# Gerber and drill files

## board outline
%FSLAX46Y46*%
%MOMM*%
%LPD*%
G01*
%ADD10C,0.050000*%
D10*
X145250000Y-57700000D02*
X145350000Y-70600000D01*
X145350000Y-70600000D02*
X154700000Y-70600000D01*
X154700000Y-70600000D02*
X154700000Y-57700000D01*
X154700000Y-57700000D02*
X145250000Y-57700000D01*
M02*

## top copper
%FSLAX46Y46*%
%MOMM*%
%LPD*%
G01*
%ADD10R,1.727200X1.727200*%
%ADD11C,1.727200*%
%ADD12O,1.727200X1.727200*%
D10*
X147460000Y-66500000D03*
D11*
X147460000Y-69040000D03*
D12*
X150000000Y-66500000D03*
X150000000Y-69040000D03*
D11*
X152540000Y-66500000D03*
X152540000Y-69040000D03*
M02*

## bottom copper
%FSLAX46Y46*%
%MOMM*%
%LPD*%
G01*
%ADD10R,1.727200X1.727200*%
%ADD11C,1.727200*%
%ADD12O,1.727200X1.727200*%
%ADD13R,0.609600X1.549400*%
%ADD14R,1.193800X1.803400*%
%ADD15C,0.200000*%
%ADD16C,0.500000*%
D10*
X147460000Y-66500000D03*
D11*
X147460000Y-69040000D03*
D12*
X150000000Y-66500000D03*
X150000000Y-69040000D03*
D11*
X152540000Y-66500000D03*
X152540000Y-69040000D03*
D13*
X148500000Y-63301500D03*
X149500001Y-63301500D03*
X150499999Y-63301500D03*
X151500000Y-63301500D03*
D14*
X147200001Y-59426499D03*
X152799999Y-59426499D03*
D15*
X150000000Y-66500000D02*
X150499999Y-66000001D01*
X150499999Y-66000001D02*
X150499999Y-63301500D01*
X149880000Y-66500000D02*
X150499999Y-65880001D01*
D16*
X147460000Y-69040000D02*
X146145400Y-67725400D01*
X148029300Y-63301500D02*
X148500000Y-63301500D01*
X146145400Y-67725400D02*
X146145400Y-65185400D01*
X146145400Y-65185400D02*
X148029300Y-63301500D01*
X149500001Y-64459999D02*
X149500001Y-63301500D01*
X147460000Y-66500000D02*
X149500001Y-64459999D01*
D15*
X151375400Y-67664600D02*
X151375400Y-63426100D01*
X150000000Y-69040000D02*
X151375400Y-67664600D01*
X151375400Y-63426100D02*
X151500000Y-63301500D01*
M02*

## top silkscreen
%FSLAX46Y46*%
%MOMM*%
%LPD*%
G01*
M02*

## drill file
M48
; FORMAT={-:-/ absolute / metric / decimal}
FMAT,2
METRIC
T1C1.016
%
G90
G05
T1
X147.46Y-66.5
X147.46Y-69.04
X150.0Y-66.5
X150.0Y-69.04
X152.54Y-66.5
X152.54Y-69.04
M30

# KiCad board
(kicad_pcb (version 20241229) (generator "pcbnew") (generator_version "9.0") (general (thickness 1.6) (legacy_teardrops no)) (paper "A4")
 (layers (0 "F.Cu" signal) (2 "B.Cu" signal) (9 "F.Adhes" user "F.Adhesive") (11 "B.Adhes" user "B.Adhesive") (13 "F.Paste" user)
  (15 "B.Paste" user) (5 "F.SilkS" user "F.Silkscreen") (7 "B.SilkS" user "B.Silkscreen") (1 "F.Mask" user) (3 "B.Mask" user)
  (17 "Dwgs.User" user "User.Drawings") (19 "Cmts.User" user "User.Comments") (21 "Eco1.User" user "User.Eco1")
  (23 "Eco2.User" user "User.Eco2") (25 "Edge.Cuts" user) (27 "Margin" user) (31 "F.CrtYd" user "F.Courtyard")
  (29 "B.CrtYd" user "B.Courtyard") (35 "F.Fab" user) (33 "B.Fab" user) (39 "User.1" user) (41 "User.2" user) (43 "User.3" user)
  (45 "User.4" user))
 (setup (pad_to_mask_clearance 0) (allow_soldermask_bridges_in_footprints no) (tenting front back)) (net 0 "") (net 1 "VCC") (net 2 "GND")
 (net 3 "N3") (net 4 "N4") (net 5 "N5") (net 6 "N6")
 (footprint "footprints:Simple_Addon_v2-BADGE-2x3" (layer "F.Cu") (at 149.94 67.75)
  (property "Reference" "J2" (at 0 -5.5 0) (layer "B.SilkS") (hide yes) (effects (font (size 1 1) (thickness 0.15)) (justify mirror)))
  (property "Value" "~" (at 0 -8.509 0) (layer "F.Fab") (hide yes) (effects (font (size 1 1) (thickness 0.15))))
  (pad "1" thru_hole rect (at -2.48 -1.25 270) (size 1.7272 1.7272) (drill 1.016) (layers "*.Cu" "*.Mask") (remove_unused_layers no)
   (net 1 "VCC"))
  (pad "2" thru_hole circle (at -2.48 1.29 270) (size 1.7272 1.7272) (drill 1.016) (layers "*.Cu" "*.Mask") (remove_unused_layers no)
   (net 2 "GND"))
  (pad "3" thru_hole oval (at 0.06 -1.25 270) (size 1.7272 1.7272) (drill 1.016) (layers "*.Cu" "*.Mask") (remove_unused_layers no)
   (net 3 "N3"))
  (pad "4" thru_hole oval (at 0.06 1.29 270) (size 1.7272 1.7272) (drill 1.016) (layers "*.Cu" "*.Mask") (remove_unused_layers no)
   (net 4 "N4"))
  (pad "5" thru_hole circle (at 2.6 -1.25 270) (size 1.7272 1.7272) (drill 1.016) (layers "*.Cu" "*.Mask") (remove_unused_layers no)
   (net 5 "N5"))
  (pad "6" thru_hole circle (at 2.6 1.29 270) (size 1.7272 1.7272) (drill 1.016) (layers "*.Cu" "*.Mask") (remove_unused_layers no)
   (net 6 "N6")))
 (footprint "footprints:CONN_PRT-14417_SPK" (layer "B.Cu") (at 150 61.2)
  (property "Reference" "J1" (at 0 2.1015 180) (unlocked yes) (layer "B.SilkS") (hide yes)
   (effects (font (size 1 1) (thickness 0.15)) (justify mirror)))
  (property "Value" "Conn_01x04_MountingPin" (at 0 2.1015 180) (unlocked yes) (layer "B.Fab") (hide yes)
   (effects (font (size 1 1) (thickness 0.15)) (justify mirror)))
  (pad "1" smd rect (at -1.5 2.1015) (size 0.6096 1.5494) (layers "B.Cu" "B.Mask" "B.Paste") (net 2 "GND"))
  (pad "2" smd rect (at -0.499999 2.1015) (size 0.6096 1.5494) (layers "B.Cu" "B.Mask" "B.Paste") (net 1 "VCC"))
  (pad "3" smd rect (at 0.499999 2.1015) (size 0.6096 1.5494) (layers "B.Cu" "B.Mask" "B.Paste") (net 3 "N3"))
  (pad "4" smd rect (at 1.5 2.1015) (size 0.6096 1.5494) (layers "B.Cu" "B.Mask" "B.Paste") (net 4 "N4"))
  (pad "5" smd rect (at -2.799999 -1.773501) (size 1.1938 1.8034) (layers "B.Cu" "B.Mask" "B.Paste"))
  (pad "6" smd rect (at 2.799999 -1.773501) (size 1.1938 1.8034) (layers "B.Cu" "B.Mask" "B.Paste")))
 (gr_line (start 145.25 57.7) (end 145.35 70.6) (stroke (width 0.05) (type default)) (layer "Edge.Cuts"))
 (gr_line (start 145.35 70.6) (end 154.7 70.6) (stroke (width 0.05) (type default)) (layer "Edge.Cuts"))
 (gr_line (start 154.7 70.6) (end 154.7 57.7) (stroke (width 0.05) (type default)) (layer "Edge.Cuts"))
 (gr_line (start 154.7 57.7) (end 145.25 57.7) (stroke (width 0.05) (type default)) (layer "Edge.Cuts"))
 (segment (start 150 66.5) (end 150.499999 66.000001) (width 0.2) (layer "B.Cu") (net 3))
 (segment (start 150.499999 66.000001) (end 150.499999 63.3015) (width 0.2) (layer "B.Cu") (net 3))
 (segment (start 149.88 66.5) (end 150.499999 65.880001) (width 0.2) (layer "B.Cu") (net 3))
 (segment (start 147.46 69.04) (end 146.1454 67.7254) (width 0.5) (layer "B.Cu") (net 2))
 (segment (start 148.0293 63.3015) (end 148.5 63.3015) (width 0.5) (layer "B.Cu") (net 2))
 (segment (start 146.1454 67.7254) (end 146.1454 65.1854) (width 0.5) (layer "B.Cu") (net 2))
 (segment (start 146.1454 65.1854) (end 148.0293 63.3015) (width 0.5) (layer "B.Cu") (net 2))
 (segment (start 149.500001 64.459999) (end 149.500001 63.3015) (width 0.5) (layer "B.Cu") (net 1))
 (segment (start 147.46 66.5) (end 149.500001 64.459999) (width 0.5) (layer "B.Cu") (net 1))
 (segment (start 151.3754 67.6646) (end 151.3754 63.4261) (width 0.2) (layer "B.Cu") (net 4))
 (segment (start 150 69.04) (end 151.3754 67.6646) (width 0.2) (layer "B.Cu") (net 4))
 (segment (start 151.3754 63.4261) (end 151.5 63.3015) (width 0.2) (layer "B.Cu") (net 4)))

